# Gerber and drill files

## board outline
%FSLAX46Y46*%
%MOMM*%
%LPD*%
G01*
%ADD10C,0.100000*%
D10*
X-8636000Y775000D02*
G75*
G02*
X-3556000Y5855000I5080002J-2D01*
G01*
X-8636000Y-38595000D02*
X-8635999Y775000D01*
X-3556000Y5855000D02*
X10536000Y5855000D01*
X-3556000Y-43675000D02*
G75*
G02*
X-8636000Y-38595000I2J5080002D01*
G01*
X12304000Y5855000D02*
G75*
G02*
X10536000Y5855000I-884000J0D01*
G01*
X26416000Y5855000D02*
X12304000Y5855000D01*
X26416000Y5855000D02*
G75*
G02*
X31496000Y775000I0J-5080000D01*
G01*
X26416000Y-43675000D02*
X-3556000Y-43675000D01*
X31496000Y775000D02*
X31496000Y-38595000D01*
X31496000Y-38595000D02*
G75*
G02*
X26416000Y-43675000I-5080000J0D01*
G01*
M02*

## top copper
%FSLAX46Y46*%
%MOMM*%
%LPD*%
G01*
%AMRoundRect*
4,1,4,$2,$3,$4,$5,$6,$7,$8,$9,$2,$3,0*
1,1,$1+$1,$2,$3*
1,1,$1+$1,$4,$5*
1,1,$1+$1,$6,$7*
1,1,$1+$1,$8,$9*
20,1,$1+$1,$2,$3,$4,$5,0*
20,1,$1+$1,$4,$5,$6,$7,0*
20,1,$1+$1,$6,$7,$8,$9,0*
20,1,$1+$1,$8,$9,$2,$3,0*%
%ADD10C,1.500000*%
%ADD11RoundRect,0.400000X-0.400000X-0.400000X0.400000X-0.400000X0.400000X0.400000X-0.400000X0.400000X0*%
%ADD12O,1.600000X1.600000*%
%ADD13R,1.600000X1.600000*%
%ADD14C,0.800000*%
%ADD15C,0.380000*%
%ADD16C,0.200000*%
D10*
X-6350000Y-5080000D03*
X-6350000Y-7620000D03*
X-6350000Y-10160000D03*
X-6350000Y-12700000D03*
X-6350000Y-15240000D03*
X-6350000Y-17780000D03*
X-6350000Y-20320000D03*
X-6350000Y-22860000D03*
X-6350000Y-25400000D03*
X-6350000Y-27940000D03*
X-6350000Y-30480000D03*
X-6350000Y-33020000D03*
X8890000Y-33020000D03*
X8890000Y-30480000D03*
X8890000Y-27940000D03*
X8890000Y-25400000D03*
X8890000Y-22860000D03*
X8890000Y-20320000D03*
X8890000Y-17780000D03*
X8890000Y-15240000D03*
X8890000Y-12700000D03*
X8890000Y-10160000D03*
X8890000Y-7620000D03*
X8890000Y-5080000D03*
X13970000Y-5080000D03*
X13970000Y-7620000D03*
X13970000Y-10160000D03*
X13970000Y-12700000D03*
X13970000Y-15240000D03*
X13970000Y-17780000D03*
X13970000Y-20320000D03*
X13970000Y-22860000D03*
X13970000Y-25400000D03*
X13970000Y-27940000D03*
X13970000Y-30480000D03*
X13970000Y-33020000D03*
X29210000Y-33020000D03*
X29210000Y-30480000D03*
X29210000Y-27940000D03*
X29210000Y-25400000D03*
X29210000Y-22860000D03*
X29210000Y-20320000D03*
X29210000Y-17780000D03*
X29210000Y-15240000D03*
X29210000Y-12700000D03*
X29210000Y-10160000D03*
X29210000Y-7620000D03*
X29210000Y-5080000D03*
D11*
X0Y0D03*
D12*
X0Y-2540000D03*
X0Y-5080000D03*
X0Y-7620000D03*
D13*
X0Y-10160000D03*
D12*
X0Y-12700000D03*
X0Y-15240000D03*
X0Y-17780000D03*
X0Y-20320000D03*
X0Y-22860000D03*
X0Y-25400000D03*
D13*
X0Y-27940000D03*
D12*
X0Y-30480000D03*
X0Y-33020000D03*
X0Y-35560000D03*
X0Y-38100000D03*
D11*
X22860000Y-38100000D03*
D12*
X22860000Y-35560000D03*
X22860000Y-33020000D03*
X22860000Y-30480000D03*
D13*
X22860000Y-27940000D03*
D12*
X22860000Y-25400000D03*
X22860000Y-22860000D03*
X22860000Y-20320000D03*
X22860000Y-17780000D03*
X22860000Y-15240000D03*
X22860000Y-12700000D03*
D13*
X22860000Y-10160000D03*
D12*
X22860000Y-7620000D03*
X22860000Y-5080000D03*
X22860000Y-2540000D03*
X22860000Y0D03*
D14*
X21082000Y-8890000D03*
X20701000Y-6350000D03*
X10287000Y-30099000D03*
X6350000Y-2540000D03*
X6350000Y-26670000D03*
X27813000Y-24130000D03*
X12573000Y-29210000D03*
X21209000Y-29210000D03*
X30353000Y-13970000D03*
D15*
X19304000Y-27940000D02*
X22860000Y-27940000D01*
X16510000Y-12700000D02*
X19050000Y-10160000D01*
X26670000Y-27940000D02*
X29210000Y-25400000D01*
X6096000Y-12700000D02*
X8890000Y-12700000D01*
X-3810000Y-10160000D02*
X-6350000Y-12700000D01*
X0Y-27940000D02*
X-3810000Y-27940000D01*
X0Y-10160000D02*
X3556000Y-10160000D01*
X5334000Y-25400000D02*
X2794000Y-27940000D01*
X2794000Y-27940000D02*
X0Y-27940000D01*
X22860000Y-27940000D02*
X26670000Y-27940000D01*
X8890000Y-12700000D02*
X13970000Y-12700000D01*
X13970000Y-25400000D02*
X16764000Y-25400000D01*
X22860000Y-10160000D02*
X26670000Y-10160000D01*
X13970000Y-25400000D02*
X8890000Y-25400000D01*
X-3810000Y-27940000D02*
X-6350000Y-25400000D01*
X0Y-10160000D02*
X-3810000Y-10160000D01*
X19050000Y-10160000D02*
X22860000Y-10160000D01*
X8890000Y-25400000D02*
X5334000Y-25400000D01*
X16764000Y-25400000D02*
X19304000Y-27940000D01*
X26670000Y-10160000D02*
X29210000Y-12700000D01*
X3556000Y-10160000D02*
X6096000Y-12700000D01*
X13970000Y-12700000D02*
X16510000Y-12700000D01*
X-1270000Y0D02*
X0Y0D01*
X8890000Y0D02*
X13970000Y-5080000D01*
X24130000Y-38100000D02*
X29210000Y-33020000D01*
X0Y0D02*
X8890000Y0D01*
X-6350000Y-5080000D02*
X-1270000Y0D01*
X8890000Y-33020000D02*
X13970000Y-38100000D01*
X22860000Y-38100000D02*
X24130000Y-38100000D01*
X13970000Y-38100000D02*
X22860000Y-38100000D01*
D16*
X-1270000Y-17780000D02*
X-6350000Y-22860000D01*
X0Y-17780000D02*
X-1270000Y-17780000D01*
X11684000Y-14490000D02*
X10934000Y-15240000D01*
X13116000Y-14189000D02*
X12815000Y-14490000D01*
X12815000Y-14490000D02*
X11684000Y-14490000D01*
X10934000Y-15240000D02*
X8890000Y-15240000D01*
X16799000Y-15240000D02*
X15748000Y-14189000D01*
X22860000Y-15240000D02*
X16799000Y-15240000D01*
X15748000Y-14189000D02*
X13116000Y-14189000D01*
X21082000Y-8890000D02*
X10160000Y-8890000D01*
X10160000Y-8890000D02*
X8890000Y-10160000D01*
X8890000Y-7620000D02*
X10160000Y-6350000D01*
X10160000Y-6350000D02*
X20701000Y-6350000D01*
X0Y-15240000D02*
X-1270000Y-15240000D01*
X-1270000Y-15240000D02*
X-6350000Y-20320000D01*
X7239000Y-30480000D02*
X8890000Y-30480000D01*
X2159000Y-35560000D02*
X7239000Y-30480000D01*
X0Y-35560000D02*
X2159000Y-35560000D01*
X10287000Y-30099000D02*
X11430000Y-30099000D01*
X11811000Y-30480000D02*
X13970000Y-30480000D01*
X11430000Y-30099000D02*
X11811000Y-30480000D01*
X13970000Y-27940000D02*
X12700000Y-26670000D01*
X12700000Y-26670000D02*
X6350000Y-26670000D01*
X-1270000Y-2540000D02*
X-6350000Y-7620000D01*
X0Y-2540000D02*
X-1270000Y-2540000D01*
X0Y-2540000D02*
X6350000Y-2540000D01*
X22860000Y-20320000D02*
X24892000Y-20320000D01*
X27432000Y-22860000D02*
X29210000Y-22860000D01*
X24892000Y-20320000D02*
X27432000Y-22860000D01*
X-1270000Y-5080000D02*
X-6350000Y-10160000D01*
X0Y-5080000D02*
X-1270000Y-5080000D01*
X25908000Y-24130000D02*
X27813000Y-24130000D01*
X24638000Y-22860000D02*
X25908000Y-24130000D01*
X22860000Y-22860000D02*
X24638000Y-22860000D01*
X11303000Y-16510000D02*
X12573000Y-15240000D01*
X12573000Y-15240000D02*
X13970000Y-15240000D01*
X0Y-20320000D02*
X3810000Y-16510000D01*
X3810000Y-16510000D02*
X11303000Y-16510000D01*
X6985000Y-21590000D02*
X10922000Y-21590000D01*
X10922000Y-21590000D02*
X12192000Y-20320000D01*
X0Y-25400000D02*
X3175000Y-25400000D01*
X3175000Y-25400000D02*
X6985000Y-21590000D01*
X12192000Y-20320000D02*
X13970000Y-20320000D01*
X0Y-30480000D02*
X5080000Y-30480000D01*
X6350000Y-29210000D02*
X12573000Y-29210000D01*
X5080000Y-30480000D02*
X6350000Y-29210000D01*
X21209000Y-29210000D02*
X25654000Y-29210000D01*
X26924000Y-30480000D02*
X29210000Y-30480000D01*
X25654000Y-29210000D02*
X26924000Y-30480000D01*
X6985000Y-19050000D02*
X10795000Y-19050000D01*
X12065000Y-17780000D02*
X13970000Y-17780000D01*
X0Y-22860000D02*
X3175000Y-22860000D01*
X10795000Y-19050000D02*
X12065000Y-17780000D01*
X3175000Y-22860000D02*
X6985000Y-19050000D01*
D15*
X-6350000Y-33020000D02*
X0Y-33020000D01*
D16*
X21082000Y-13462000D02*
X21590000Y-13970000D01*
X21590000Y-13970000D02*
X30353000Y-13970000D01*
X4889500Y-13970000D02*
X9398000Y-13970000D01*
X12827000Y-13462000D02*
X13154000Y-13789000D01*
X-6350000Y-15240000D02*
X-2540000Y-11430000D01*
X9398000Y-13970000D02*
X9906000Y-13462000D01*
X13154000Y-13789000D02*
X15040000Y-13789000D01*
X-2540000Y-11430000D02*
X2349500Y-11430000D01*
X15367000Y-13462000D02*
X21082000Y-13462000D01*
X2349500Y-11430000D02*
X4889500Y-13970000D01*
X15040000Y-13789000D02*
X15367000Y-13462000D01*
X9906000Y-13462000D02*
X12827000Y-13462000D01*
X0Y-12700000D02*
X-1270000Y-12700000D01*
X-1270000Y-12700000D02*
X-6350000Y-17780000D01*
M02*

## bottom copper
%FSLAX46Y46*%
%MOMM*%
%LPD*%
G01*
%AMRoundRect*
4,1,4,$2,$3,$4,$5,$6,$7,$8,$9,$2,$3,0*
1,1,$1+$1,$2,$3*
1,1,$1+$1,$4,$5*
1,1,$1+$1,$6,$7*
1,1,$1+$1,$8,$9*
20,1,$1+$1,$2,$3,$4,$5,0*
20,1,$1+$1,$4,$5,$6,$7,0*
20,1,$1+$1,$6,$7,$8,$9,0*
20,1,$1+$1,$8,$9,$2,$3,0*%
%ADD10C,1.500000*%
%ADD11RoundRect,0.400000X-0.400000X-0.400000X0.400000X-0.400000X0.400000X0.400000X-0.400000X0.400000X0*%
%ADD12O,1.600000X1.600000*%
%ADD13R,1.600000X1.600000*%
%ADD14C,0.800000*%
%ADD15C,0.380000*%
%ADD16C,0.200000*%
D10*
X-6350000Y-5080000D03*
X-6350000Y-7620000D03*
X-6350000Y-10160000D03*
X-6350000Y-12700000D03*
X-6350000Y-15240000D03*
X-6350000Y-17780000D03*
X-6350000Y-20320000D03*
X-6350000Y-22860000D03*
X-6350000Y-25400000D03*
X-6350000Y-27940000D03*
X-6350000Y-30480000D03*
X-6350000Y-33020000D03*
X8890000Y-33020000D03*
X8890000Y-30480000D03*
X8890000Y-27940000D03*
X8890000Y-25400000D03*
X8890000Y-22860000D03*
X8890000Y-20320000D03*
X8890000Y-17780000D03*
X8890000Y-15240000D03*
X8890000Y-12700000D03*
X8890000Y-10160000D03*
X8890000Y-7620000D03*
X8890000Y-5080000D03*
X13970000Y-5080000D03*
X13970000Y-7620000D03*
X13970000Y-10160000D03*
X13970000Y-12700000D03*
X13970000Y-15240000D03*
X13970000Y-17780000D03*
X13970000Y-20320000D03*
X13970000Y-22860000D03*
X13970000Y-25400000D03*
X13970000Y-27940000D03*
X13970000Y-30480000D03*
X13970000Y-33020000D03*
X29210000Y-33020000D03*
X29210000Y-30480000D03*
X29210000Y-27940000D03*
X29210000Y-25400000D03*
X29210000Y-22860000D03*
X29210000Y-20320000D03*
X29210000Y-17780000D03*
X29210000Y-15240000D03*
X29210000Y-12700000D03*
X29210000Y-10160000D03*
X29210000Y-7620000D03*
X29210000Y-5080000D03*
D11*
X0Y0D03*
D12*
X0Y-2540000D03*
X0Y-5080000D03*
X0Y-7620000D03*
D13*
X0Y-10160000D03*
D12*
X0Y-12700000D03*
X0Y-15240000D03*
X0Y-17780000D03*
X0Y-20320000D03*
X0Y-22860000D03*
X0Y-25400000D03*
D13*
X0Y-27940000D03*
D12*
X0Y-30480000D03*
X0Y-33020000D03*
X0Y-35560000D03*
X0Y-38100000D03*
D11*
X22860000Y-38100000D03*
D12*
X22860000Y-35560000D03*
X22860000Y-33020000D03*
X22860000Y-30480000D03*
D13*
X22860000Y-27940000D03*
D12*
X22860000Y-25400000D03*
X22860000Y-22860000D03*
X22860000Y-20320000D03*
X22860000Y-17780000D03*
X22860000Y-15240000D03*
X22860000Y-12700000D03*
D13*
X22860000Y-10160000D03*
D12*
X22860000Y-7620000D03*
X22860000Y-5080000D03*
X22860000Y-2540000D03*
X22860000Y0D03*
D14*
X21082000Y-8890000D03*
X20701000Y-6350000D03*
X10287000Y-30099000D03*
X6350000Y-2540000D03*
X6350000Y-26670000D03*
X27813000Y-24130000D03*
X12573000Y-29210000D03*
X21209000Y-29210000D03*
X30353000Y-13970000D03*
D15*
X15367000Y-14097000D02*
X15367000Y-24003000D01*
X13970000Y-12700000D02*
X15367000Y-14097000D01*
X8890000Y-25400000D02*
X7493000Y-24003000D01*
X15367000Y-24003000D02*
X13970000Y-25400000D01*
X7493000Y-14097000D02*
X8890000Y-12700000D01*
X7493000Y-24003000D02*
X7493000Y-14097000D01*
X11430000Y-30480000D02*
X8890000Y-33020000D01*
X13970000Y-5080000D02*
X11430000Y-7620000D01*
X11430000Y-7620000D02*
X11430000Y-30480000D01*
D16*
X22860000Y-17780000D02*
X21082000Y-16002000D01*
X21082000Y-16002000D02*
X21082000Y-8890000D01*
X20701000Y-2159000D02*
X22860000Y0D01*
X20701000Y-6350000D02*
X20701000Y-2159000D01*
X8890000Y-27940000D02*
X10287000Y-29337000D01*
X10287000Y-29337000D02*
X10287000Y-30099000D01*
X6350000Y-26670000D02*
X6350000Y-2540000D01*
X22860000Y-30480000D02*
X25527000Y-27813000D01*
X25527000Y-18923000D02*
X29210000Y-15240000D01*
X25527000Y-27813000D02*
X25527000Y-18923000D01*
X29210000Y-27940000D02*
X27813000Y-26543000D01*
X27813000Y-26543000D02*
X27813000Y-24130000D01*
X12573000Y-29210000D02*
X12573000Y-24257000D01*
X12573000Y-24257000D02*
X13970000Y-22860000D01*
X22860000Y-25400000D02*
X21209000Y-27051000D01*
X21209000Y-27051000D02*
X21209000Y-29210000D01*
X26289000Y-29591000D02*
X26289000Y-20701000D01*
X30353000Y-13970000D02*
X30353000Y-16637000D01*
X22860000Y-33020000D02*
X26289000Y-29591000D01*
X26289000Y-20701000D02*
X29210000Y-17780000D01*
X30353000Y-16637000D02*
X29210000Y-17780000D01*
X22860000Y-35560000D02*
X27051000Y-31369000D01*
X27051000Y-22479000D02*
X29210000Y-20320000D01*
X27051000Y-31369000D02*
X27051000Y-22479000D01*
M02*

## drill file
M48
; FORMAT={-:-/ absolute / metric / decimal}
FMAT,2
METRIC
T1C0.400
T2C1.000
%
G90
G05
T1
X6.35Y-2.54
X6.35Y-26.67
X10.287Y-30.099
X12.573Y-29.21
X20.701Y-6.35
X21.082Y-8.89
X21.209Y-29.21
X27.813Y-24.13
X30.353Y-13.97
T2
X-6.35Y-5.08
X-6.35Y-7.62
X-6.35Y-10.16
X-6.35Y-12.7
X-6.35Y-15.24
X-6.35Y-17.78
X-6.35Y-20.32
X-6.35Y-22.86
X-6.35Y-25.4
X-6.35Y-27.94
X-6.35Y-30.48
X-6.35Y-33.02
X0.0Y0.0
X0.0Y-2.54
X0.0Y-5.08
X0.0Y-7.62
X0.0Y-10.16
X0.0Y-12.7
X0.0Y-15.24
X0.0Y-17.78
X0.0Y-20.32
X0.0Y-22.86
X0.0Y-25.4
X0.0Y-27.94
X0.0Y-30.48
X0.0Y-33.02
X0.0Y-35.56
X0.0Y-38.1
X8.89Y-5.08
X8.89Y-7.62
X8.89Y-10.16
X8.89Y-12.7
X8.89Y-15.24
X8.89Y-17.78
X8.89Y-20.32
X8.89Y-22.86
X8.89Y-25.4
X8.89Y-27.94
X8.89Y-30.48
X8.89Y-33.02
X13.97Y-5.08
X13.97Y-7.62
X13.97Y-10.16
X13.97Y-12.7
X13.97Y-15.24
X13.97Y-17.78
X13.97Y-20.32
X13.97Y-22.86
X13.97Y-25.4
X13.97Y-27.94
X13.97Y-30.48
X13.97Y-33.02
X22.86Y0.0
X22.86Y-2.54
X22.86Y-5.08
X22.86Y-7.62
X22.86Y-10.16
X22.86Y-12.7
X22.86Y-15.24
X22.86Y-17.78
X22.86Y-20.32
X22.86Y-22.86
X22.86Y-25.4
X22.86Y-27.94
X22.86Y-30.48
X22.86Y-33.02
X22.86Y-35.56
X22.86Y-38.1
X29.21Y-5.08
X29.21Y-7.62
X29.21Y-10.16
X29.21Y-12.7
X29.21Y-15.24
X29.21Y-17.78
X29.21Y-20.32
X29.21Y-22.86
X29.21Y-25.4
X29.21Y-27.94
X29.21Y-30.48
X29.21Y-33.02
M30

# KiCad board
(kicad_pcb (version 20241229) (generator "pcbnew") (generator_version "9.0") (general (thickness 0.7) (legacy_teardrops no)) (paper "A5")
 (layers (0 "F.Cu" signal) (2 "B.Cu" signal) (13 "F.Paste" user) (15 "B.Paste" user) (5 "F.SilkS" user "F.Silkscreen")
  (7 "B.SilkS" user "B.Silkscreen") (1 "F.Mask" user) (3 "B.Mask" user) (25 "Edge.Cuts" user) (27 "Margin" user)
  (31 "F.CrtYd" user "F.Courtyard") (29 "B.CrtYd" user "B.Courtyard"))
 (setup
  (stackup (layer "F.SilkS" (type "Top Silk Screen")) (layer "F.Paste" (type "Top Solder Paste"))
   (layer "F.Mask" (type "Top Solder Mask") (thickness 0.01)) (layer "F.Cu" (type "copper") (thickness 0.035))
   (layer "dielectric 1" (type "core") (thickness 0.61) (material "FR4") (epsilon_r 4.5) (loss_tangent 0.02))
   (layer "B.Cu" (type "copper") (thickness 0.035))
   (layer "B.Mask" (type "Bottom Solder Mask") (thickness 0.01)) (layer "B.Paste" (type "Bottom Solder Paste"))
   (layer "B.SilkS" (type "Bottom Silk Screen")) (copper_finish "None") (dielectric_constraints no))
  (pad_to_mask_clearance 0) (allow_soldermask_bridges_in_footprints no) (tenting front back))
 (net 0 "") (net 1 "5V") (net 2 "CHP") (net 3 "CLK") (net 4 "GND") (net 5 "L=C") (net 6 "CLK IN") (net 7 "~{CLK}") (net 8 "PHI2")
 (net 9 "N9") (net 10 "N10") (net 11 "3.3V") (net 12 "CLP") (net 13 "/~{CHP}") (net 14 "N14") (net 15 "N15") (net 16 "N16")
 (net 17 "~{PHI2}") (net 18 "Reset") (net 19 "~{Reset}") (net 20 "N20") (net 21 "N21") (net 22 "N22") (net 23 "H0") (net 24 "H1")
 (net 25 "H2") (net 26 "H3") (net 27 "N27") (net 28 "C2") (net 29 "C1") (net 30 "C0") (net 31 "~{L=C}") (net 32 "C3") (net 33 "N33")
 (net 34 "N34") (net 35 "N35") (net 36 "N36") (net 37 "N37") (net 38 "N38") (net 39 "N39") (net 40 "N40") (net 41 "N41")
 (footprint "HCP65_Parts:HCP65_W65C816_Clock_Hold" (layer "F.Cu") (at -6.35 5.08)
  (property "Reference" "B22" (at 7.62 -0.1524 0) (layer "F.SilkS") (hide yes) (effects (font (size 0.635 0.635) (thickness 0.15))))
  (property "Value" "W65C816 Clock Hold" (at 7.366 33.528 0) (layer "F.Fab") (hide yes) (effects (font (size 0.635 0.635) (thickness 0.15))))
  (pad "1" thru_hole circle (at 0 0) (size 1.5 1.5) (drill 1) (layers "*.Cu" "*.Mask") (remove_unused_layers no) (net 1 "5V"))
  (pad "2" thru_hole circle (at 0 2.54) (size 1.5 1.5) (drill 1) (layers "*.Cu" "*.Mask") (remove_unused_layers no) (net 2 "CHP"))
  (pad "3" thru_hole circle (at 0 5.08) (size 1.5 1.5) (drill 1) (layers "*.Cu" "*.Mask") (remove_unused_layers no) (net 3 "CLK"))
  (pad "4" thru_hole circle (at 0 7.62) (size 1.5 1.5) (drill 1) (layers "*.Cu" "*.Mask") (remove_unused_layers no) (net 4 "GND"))
  (pad "5" thru_hole circle (at 0 10.16) (size 1.5 1.5) (drill 1) (layers "*.Cu" "*.Mask") (remove_unused_layers no) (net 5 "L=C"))
  (pad "6" thru_hole circle (at 0 12.7) (size 1.5 1.5) (drill 1) (layers "*.Cu" "*.Mask") (remove_unused_layers no) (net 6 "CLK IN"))
  (pad "7" thru_hole circle (at 0 15.24) (size 1.5 1.5) (drill 1) (layers "*.Cu" "*.Mask") (remove_unused_layers no) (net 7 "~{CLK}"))
  (pad "8" thru_hole circle (at 0 17.78) (size 1.5 1.5) (drill 1) (layers "*.Cu" "*.Mask") (remove_unused_layers no) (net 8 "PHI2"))
  (pad "9" thru_hole circle (at 0 20.32) (size 1.5 1.5) (drill 1) (layers "*.Cu" "*.Mask") (remove_unused_layers no) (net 4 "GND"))
  (pad "10" thru_hole circle (at 0 22.86) (size 1.5 1.5) (drill 1) (layers "*.Cu" "*.Mask") (remove_unused_layers no) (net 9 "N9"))
  (pad "11" thru_hole circle (at 0 25.4) (size 1.5 1.5) (drill 1) (layers "*.Cu" "*.Mask") (remove_unused_layers no) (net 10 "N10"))
  (pad "12" thru_hole circle (at 0 27.94) (size 1.5 1.5) (drill 1) (layers "*.Cu" "*.Mask") (remove_unused_layers no) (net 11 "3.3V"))
  (pad "13" thru_hole circle (at 15.24 27.94) (size 1.5 1.5) (drill 1) (layers "*.Cu" "*.Mask") (remove_unused_layers no) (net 1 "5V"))
  (pad "14" thru_hole circle (at 15.24 25.4) (size 1.5 1.5) (drill 1) (layers "*.Cu" "*.Mask") (remove_unused_layers no) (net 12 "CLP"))
  (pad "15" thru_hole circle (at 15.24 22.86) (size 1.5 1.5) (drill 1) (layers "*.Cu" "*.Mask") (remove_unused_layers no) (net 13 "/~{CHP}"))
  (pad "16" thru_hole circle (at 15.24 20.32) (size 1.5 1.5) (drill 1) (layers "*.Cu" "*.Mask") (remove_unused_layers no) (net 4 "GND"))
  (pad "17" thru_hole circle (at 15.24 17.78) (size 1.5 1.5) (drill 1) (layers "*.Cu" "*.Mask") (remove_unused_layers no) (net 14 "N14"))
  (pad "18" thru_hole circle (at 15.24 15.24) (size 1.5 1.5) (drill 1) (layers "*.Cu" "*.Mask") (remove_unused_layers no) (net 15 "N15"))
  (pad "19" thru_hole circle (at 15.24 12.7) (size 1.5 1.5) (drill 1) (layers "*.Cu" "*.Mask") (remove_unused_layers no) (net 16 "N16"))
  (pad "20" thru_hole circle (at 15.24 10.16) (size 1.5 1.5) (drill 1) (layers "*.Cu" "*.Mask") (remove_unused_layers no) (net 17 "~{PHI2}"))
  (pad "21" thru_hole circle (at 15.24 7.62) (size 1.5 1.5) (drill 1) (layers "*.Cu" "*.Mask") (remove_unused_layers no) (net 4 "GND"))
  (pad "22" thru_hole circle (at 15.24 5.08) (size 1.5 1.5) (drill 1) (layers "*.Cu" "*.Mask") (remove_unused_layers no) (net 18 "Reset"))
  (pad "23" thru_hole circle (at 15.24 2.54) (size 1.5 1.5) (drill 1) (layers "*.Cu" "*.Mask") (remove_unused_layers no) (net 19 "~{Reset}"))
  (pad "24" thru_hole circle (at 15.24 0) (size 1.5 1.5) (drill 1) (layers "*.Cu" "*.Mask") (remove_unused_layers no) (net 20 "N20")))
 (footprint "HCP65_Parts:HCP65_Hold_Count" (layer "F.Cu") (at 13.97 5.08)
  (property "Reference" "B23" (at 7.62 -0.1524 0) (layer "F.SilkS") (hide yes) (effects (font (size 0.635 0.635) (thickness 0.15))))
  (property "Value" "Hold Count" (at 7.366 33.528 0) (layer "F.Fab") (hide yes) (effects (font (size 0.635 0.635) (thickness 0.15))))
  (pad "1" thru_hole circle (at 0 0) (size 1.5 1.5) (drill 1) (layers "*.Cu" "*.Mask") (remove_unused_layers no) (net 1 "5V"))
  (pad "2" thru_hole circle (at 0 2.54) (size 1.5 1.5) (drill 1) (layers "*.Cu" "*.Mask") (remove_unused_layers no) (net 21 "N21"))
  (pad "3" thru_hole circle (at 0 5.08) (size 1.5 1.5) (drill 1) (layers "*.Cu" "*.Mask") (remove_unused_layers no) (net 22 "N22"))
  (pad "4" thru_hole circle (at 0 7.62) (size 1.5 1.5) (drill 1) (layers "*.Cu" "*.Mask") (remove_unused_layers no) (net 4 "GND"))
  (pad "5" thru_hole circle (at 0 10.16) (size 1.5 1.5) (drill 1) (layers "*.Cu" "*.Mask") (remove_unused_layers no) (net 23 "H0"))
  (pad "6" thru_hole circle (at 0 12.7) (size 1.5 1.5) (drill 1) (layers "*.Cu" "*.Mask") (remove_unused_layers no) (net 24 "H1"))
  (pad "7" thru_hole circle (at 0 15.24) (size 1.5 1.5) (drill 1) (layers "*.Cu" "*.Mask") (remove_unused_layers no) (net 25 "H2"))
  (pad "8" thru_hole circle (at 0 17.78) (size 1.5 1.5) (drill 1) (layers "*.Cu" "*.Mask") (remove_unused_layers no) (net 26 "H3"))
  (pad "9" thru_hole circle (at 0 20.32) (size 1.5 1.5) (drill 1) (layers "*.Cu" "*.Mask") (remove_unused_layers no) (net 4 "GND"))
  (pad "10" thru_hole circle (at 0 22.86) (size 1.5 1.5) (drill 1) (layers "*.Cu" "*.Mask") (remove_unused_layers no) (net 2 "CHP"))
  (pad "11" thru_hole circle (at 0 25.4) (size 1.5 1.5) (drill 1) (layers "*.Cu" "*.Mask") (remove_unused_layers no) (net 13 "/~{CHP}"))
  (pad "12" thru_hole circle (at 0 27.94) (size 1.5 1.5) (drill 1) (layers "*.Cu" "*.Mask") (remove_unused_layers no) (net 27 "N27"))
  (pad "13" thru_hole circle (at 15.24 27.94) (size 1.5 1.5) (drill 1) (layers "*.Cu" "*.Mask") (remove_unused_layers no) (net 1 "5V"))
  (pad "14" thru_hole circle (at 15.24 25.4) (size 1.5 1.5) (drill 1) (layers "*.Cu" "*.Mask") (remove_unused_layers no) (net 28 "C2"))
  (pad "15" thru_hole circle (at 15.24 22.86) (size 1.5 1.5) (drill 1) (layers "*.Cu" "*.Mask") (remove_unused_layers no) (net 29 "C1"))
  (pad "16" thru_hole circle (at 15.24 20.32) (size 1.5 1.5) (drill 1) (layers "*.Cu" "*.Mask") (remove_unused_layers no) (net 4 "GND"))
  (pad "17" thru_hole circle (at 15.24 17.78) (size 1.5 1.5) (drill 1) (layers "*.Cu" "*.Mask") (remove_unused_layers no) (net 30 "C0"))
  (pad "18" thru_hole circle (at 15.24 15.24) (size 1.5 1.5) (drill 1) (layers "*.Cu" "*.Mask") (remove_unused_layers no) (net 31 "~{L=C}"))
  (pad "19" thru_hole circle (at 15.24 12.7) (size 1.5 1.5) (drill 1) (layers "*.Cu" "*.Mask") (remove_unused_layers no) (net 5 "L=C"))
  (pad "20" thru_hole circle (at 15.24 10.16) (size 1.5 1.5) (drill 1) (layers "*.Cu" "*.Mask") (remove_unused_layers no) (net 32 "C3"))
  (pad "21" thru_hole circle (at 15.24 7.62) (size 1.5 1.5) (drill 1) (layers "*.Cu" "*.Mask") (remove_unused_layers no) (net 4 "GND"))
  (pad "22" thru_hole circle (at 15.24 5.08) (size 1.5 1.5) (drill 1) (layers "*.Cu" "*.Mask") (remove_unused_layers no) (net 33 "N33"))
  (pad "23" thru_hole circle (at 15.24 2.54) (size 1.5 1.5) (drill 1) (layers "*.Cu" "*.Mask") (remove_unused_layers no) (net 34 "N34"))
  (pad "24" thru_hole circle (at 15.24 0) (size 1.5 1.5) (drill 1) (layers "*.Cu" "*.Mask") (remove_unused_layers no) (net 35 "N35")))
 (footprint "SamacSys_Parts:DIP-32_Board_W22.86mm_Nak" (layer "F.Cu") (at 0 0)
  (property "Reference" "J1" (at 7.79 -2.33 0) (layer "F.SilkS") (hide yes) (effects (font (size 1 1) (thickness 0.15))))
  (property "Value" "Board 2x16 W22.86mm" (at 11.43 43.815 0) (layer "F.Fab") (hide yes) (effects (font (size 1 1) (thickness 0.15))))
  (pad "1" thru_hole roundrect (at 0 0) (size 1.6 1.6) (drill 1) (layers "*.Cu" "*.Mask") (remove_unused_layers no) (roundrect_rratio 0.25)
   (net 1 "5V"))
  (pad "2" thru_hole oval (at 0 2.54) (size 1.6 1.6) (drill 1) (layers "*.Cu" "*.Mask") (remove_unused_layers no) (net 2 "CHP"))
  (pad "3" thru_hole oval (at 0 5.08) (size 1.6 1.6) (drill 1) (layers "*.Cu" "*.Mask") (remove_unused_layers no) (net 3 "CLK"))
  (pad "4" thru_hole oval (at 0 7.62) (size 1.6 1.6) (drill 1) (layers "*.Cu" "*.Mask") (remove_unused_layers no) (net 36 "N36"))
  (pad "5" thru_hole rect (at 0 10.16) (size 1.6 1.6) (drill 1) (layers "*.Cu" "*.Mask") (remove_unused_layers no) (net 4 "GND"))
  (pad "6" thru_hole oval (at 0 12.7) (size 1.6 1.6) (drill 1) (layers "*.Cu" "*.Mask") (remove_unused_layers no) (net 6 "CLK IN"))
  (pad "7" thru_hole oval (at 0 15.24) (size 1.6 1.6) (drill 1) (layers "*.Cu" "*.Mask") (remove_unused_layers no) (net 7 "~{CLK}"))
  (pad "8" thru_hole oval (at 0 17.78) (size 1.6 1.6) (drill 1) (layers "*.Cu" "*.Mask") (remove_unused_layers no) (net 8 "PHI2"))
  (pad "9" thru_hole oval (at 0 20.32) (size 1.6 1.6) (drill 1) (layers "*.Cu" "*.Mask") (remove_unused_layers no) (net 23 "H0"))
  (pad "10" thru_hole oval (at 0 22.86) (size 1.6 1.6) (drill 1) (layers "*.Cu" "*.Mask") (remove_unused_layers no) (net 24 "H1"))
  (pad "11" thru_hole oval (at 0 25.4) (size 1.6 1.6) (drill 1) (layers "*.Cu" "*.Mask") (remove_unused_layers no) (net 25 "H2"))
  (pad "12" thru_hole rect (at 0 27.94) (size 1.6 1.6) (drill 1) (layers "*.Cu" "*.Mask") (remove_unused_layers no) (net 4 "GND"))
  (pad "13" thru_hole oval (at 0 30.48) (size 1.6 1.6) (drill 1) (layers "*.Cu" "*.Mask") (remove_unused_layers no) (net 26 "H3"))
  (pad "14" thru_hole oval (at 0 33.02) (size 1.6 1.6) (drill 1) (layers "*.Cu" "*.Mask") (remove_unused_layers no) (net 11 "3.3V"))
  (pad "15" thru_hole oval (at 0 35.56) (size 1.6 1.6) (drill 1) (layers "*.Cu" "*.Mask") (remove_unused_layers no) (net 12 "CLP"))
  (pad "16" thru_hole oval (at 0 38.1) (size 1.6 1.6) (drill 1) (layers "*.Cu" "*.Mask") (remove_unused_layers no) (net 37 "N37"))
  (pad "17" thru_hole roundrect (at 22.86 38.1) (size 1.6 1.6) (drill 1) (layers "*.Cu" "*.Mask") (remove_unused_layers no)
   (roundrect_rratio 0.25) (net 1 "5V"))
  (pad "18" thru_hole oval (at 22.86 35.56) (size 1.6 1.6) (drill 1) (layers "*.Cu" "*.Mask") (remove_unused_layers no) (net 31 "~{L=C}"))
  (pad "19" thru_hole oval (at 22.86 33.02) (size 1.6 1.6) (drill 1) (layers "*.Cu" "*.Mask") (remove_unused_layers no) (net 5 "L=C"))
  (pad "20" thru_hole oval (at 22.86 30.48) (size 1.6 1.6) (drill 1) (layers "*.Cu" "*.Mask") (remove_unused_layers no) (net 32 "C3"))
  (pad "21" thru_hole rect (at 22.86 27.94) (size 1.6 1.6) (drill 1) (layers "*.Cu" "*.Mask") (remove_unused_layers no) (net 4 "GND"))
  (pad "22" thru_hole oval (at 22.86 25.4) (size 1.6 1.6) (drill 1) (layers "*.Cu" "*.Mask") (remove_unused_layers no) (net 28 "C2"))
  (pad "23" thru_hole oval (at 22.86 22.86) (size 1.6 1.6) (drill 1) (layers "*.Cu" "*.Mask") (remove_unused_layers no) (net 29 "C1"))
  (pad "24" thru_hole oval (at 22.86 20.32) (size 1.6 1.6) (drill 1) (layers "*.Cu" "*.Mask") (remove_unused_layers no) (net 30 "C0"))
  (pad "25" thru_hole oval (at 22.86 17.78) (size 1.6 1.6) (drill 1) (layers "*.Cu" "*.Mask") (remove_unused_layers no) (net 18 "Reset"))
  (pad "26" thru_hole oval (at 22.86 15.24) (size 1.6 1.6) (drill 1) (layers "*.Cu" "*.Mask") (remove_unused_layers no) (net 17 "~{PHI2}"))
  (pad "27" thru_hole oval (at 22.86 12.7) (size 1.6 1.6) (drill 1) (layers "*.Cu" "*.Mask") (remove_unused_layers no) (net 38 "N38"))
  (pad "28" thru_hole rect (at 22.86 10.16) (size 1.6 1.6) (drill 1) (layers "*.Cu" "*.Mask") (remove_unused_layers no) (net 4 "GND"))
  (pad "29" thru_hole oval (at 22.86 7.62) (size 1.6 1.6) (drill 1) (layers "*.Cu" "*.Mask") (remove_unused_layers no) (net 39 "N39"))
  (pad "30" thru_hole oval (at 22.86 5.08) (size 1.6 1.6) (drill 1) (layers "*.Cu" "*.Mask") (remove_unused_layers no) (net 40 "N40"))
  (pad "31" thru_hole oval (at 22.86 2.54) (size 1.6 1.6) (drill 1) (layers "*.Cu" "*.Mask") (remove_unused_layers no) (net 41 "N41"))
  (pad "32" thru_hole oval (at 22.86 0) (size 1.6 1.6) (drill 1) (layers "*.Cu" "*.Mask") (remove_unused_layers no) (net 19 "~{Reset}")))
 (gr_arc (start -8.636 -0.775) (mid -7.148102 -4.367102) (end -3.556 -5.855) (stroke (width 0.1) (type default)) (layer "Edge.Cuts"))
 (gr_line (start -8.636 38.595) (end -8.635999 -0.775) (stroke (width 0.1) (type default)) (layer "Edge.Cuts"))
 (gr_line (start -3.556 -5.855) (end 10.536 -5.855) (stroke (width 0.1) (type default)) (layer "Edge.Cuts"))
 (gr_arc (start -3.556 43.675) (mid -7.148102 42.187102) (end -8.636 38.595) (stroke (width 0.1) (type default)) (layer "Edge.Cuts"))
 (gr_arc (start 12.304 -5.855) (mid 11.42 -4.971) (end 10.536 -5.855) (stroke (width 0.1) (type solid)) (layer "Edge.Cuts"))
 (gr_line (start 26.416 -5.855) (end 12.304 -5.855) (stroke (width 0.1) (type solid)) (layer "Edge.Cuts"))
 (gr_arc (start 26.416 -5.855) (mid 30.008102 -4.367102) (end 31.496 -0.775) (stroke (width 0.1) (type default)) (layer "Edge.Cuts"))
 (gr_line (start 26.416 43.675) (end -3.556 43.675) (stroke (width 0.1) (type default)) (layer "Edge.Cuts"))
 (gr_line (start 31.496 -0.775) (end 31.496 38.595) (stroke (width 0.1) (type default)) (layer "Edge.Cuts"))
 (gr_arc (start 31.496 38.595) (mid 30.008102 42.187102) (end 26.416 43.675) (stroke (width 0.1) (type default)) (layer "Edge.Cuts"))
 (segment (start 19.304 27.94) (end 22.86 27.94) (width 0.38) (layer "F.Cu") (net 4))
 (segment (start 16.51 12.7) (end 19.05 10.16) (width 0.38) (layer "F.Cu") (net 4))
 (segment (start 26.67 27.94) (end 29.21 25.4) (width 0.38) (layer "F.Cu") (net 4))
 (segment (start 6.096 12.7) (end 8.89 12.7) (width 0.38) (layer "F.Cu") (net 4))
 (segment (start -3.81 10.16) (end -6.35 12.7) (width 0.38) (layer "F.Cu") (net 4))
 (segment (start 0 27.94) (end -3.81 27.94) (width 0.38) (layer "F.Cu") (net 4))
 (segment (start 0 10.16) (end 3.556 10.16) (width 0.38) (layer "F.Cu") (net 4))
 (segment (start 5.334 25.4) (end 2.794 27.94) (width 0.38) (layer "F.Cu") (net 4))
 (segment (start 2.794 27.94) (end 0 27.94) (width 0.38) (layer "F.Cu") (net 4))
 (segment (start 22.86 27.94) (end 26.67 27.94) (width 0.38) (layer "F.Cu") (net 4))
 (segment (start 8.89 12.7) (end 13.97 12.7) (width 0.38) (layer "F.Cu") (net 4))
 (segment (start 13.97 25.4) (end 16.764 25.4) (width 0.38) (layer "F.Cu") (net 4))
 (segment (start 22.86 10.16) (end 26.67 10.16) (width 0.38) (layer "F.Cu") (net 4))
 (segment (start 13.97 25.4) (end 8.89 25.4) (width 0.38) (layer "F.Cu") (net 4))
 (segment (start -3.81 27.94) (end -6.35 25.4) (width 0.38) (layer "F.Cu") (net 4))
 (segment (start 0 10.16) (end -3.81 10.16) (width 0.38) (layer "F.Cu") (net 4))
 (segment (start 19.05 10.16) (end 22.86 10.16) (width 0.38) (layer "F.Cu") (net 4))
 (segment (start 8.89 25.4) (end 5.334 25.4) (width 0.38) (layer "F.Cu") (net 4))
 (segment (start 16.764 25.4) (end 19.304 27.94) (width 0.38) (layer "F.Cu") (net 4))
 (segment (start 26.67 10.16) (end 29.21 12.7) (width 0.38) (layer "F.Cu") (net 4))
 (segment (start 3.556 10.16) (end 6.096 12.7) (width 0.38) (layer "F.Cu") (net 4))
 (segment (start 13.97 12.7) (end 16.51 12.7) (width 0.38) (layer "F.Cu") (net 4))
 (segment (start 15.367 14.097) (end 15.367 24.003) (width 0.38) (layer "B.Cu") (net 4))
 (segment (start 13.97 12.7) (end 15.367 14.097) (width 0.38) (layer "B.Cu") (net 4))
 (segment (start 8.89 25.4) (end 7.493 24.003) (width 0.38) (layer "B.Cu") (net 4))
 (segment (start 15.367 24.003) (end 13.97 25.4) (width 0.38) (layer "B.Cu") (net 4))
 (segment (start 7.493 14.097) (end 8.89 12.7) (width 0.38) (layer "B.Cu") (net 4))
 (segment (start 7.493 24.003) (end 7.493 14.097) (width 0.38) (layer "B.Cu") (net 4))
 (segment (start -1.27 0) (end 0 0) (width 0.38) (layer "F.Cu") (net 1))
 (segment (start 8.89 0) (end 13.97 5.08) (width 0.38) (layer "F.Cu") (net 1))
 (segment (start 24.13 38.1) (end 29.21 33.02) (width 0.38) (layer "F.Cu") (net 1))
 (segment (start 0 0) (end 8.89 0) (width 0.38) (layer "F.Cu") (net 1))
 (segment (start -6.35 5.08) (end -1.27 0) (width 0.38) (layer "F.Cu") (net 1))
 (segment (start 8.89 33.02) (end 13.97 38.1) (width 0.38) (layer "F.Cu") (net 1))
 (segment (start 22.86 38.1) (end 24.13 38.1) (width 0.38) (layer "F.Cu") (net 1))
 (segment (start 13.97 38.1) (end 22.86 38.1) (width 0.38) (layer "F.Cu") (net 1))
 (segment (start 11.43 30.48) (end 8.89 33.02) (width 0.38) (layer "B.Cu") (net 1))
 (segment (start 13.97 5.08) (end 11.43 7.62) (width 0.38) (layer "B.Cu") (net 1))
 (segment (start 11.43 7.62) (end 11.43 30.48) (width 0.38) (layer "B.Cu") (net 1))
 (segment (start -1.27 17.78) (end -6.35 22.86) (width 0.2) (layer "F.Cu") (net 8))
 (segment (start 0 17.78) (end -1.27 17.78) (width 0.2) (layer "F.Cu") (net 8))
 (segment (start 11.684 14.49) (end 10.934 15.24) (width 0.2) (layer "F.Cu") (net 17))
 (segment (start 13.116 14.189) (end 12.815 14.49) (width 0.2) (layer "F.Cu") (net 17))
 (segment (start 12.815 14.49) (end 11.684 14.49) (width 0.2) (layer "F.Cu") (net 17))
 (segment (start 10.934 15.24) (end 8.89 15.24) (width 0.2) (layer "F.Cu") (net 17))
 (segment (start 16.799 15.24) (end 15.748 14.189) (width 0.2) (layer "F.Cu") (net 17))
 (segment (start 22.86 15.24) (end 16.799 15.24) (width 0.2) (layer "F.Cu") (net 17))
 (segment (start 15.748 14.189) (end 13.116 14.189) (width 0.2) (layer "F.Cu") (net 17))
 (segment (start 21.082 8.89) (end 10.16 8.89) (width 0.2) (layer "F.Cu") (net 18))
 (segment (start 10.16 8.89) (end 8.89 10.16) (width 0.2) (layer "F.Cu") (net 18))
 (via (at 21.082 8.89) (size 0.8) (drill 0.4) (layers "F.Cu" "B.Cu") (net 18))
 (segment (start 22.86 17.78) (end 21.082 16.002) (width 0.2) (layer "B.Cu") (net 18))
 (segment (start 21.082 16.002) (end 21.082 8.89) (width 0.2) (layer "B.Cu") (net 18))
 (segment (start 8.89 7.62) (end 10.16 6.35) (width 0.2) (layer "F.Cu") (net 19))
 (segment (start 10.16 6.35) (end 20.701 6.35) (width 0.2) (layer "F.Cu") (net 19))
 (via (at 20.701 6.35) (size 0.8) (drill 0.4) (layers "F.Cu" "B.Cu") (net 19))
 (segment (start 20.701 2.159) (end 22.86 0) (width 0.2) (layer "B.Cu") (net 19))
 (segment (start 20.701 6.35) (end 20.701 2.159) (width 0.2) (layer "B.Cu") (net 19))
 (segment (start 0 15.24) (end -1.27 15.24) (width 0.2) (layer "F.Cu") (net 7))
 (segment (start -1.27 15.24) (end -6.35 20.32) (width 0.2) (layer "F.Cu") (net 7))
 (segment (start 7.239 30.48) (end 8.89 30.48) (width 0.2) (layer "F.Cu") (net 12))
 (segment (start 2.159 35.56) (end 7.239 30.48) (width 0.2) (layer "F.Cu") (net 12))
 (segment (start 0 35.56) (end 2.159 35.56) (width 0.2) (layer "F.Cu") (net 12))
 (segment (start 10.287 30.099) (end 11.43 30.099) (width 0.2) (layer "F.Cu") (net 13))
 (segment (start 11.811 30.48) (end 13.97 30.48) (width 0.2) (layer "F.Cu") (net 13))
 (segment (start 11.43 30.099) (end 11.811 30.48) (width 0.2) (layer "F.Cu") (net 13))
 (via (at 10.287 30.099) (size 0.8) (drill 0.4) (layers "F.Cu" "B.Cu") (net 13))
 (segment (start 8.89 27.94) (end 10.287 29.337) (width 0.2) (layer "B.Cu") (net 13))
 (segment (start 10.287 29.337) (end 10.287 30.099) (width 0.2) (layer "B.Cu") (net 13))
 (segment (start 13.97 27.94) (end 12.7 26.67) (width 0.2) (layer "F.Cu") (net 2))
 (segment (start 12.7 26.67) (end 6.35 26.67) (width 0.2) (layer "F.Cu") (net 2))
 (segment (start -1.27 2.54) (end -6.35 7.62) (width 0.2) (layer "F.Cu") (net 2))
 (segment (start 0 2.54) (end -1.27 2.54) (width 0.2) (layer "F.Cu") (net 2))
 (segment (start 0 2.54) (end 6.35 2.54) (width 0.2) (layer "F.Cu") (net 2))
 (via (at 6.35 2.54) (size 0.8) (drill 0.4) (layers "F.Cu" "B.Cu") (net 2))
 (via (at 6.35 26.67) (size 0.8) (drill 0.4) (layers "F.Cu" "B.Cu") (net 2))
 (segment (start 6.35 26.67) (end 6.35 2.54) (width 0.2) (layer "B.Cu") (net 2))
 (segment (start 22.86 20.32) (end 24.892 20.32) (width 0.2) (layer "F.Cu") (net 30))
 (segment (start 27.432 22.86) (end 29.21 22.86) (width 0.2) (layer "F.Cu") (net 30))
 (segment (start 24.892 20.32) (end 27.432 22.86) (width 0.2) (layer "F.Cu") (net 30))
 (segment (start -1.27 5.08) (end -6.35 10.16) (width 0.2) (layer "F.Cu") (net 3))
 (segment (start 0 5.08) (end -1.27 5.08) (width 0.2) (layer "F.Cu") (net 3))
 (segment (start 22.86 30.48) (end 25.527 27.813) (width 0.2) (layer "B.Cu") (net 32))
 (segment (start 25.527 18.923) (end 29.21 15.24) (width 0.2) (layer "B.Cu") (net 32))
 (segment (start 25.527 27.813) (end 25.527 18.923) (width 0.2) (layer "B.Cu") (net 32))
 (segment (start 25.908 24.13) (end 27.813 24.13) (width 0.2) (layer "F.Cu") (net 29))
 (segment (start 24.638 22.86) (end 25.908 24.13) (width 0.2) (layer "F.Cu") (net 29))
 (segment (start 22.86 22.86) (end 24.638 22.86) (width 0.2) (layer "F.Cu") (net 29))
 (via (at 27.813 24.13) (size 0.8) (drill 0.4) (layers "F.Cu" "B.Cu") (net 29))
 (segment (start 29.21 27.94) (end 27.813 26.543) (width 0.2) (layer "B.Cu") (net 29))
 (segment (start 27.813 26.543) (end 27.813 24.13) (width 0.2) (layer "B.Cu") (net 29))
 (segment (start 11.303 16.51) (end 12.573 15.24) (width 0.2) (layer "F.Cu") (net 23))
 (segment (start 12.573 15.24) (end 13.97 15.24) (width 0.2) (layer "F.Cu") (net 23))
 (segment (start 0 20.32) (end 3.81 16.51) (width 0.2) (layer "F.Cu") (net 23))
 (segment (start 3.81 16.51) (end 11.303 16.51) (width 0.2) (layer "F.Cu") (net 23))
 (segment (start 6.985 21.59) (end 10.922 21.59) (width 0.2) (layer "F.Cu") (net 25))
 (segment (start 10.922 21.59) (end 12.192 20.32) (width 0.2) (layer "F.Cu") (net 25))
 (segment (start 0 25.4) (end 3.175 25.4) (width 0.2) (layer "F.Cu") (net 25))
 (segment (start 3.175 25.4) (end 6.985 21.59) (width 0.2) (layer "F.Cu") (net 25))
 (segment (start 12.192 20.32) (end 13.97 20.32) (width 0.2) (layer "F.Cu") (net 25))
 (segment (start 0 30.48) (end 5.08 30.48) (width 0.2) (layer "F.Cu") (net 26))
 (segment (start 6.35 29.21) (end 12.573 29.21) (width 0.2) (layer "F.Cu") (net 26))
 (segment (start 5.08 30.48) (end 6.35 29.21) (width 0.2) (layer "F.Cu") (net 26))
 (via (at 12.573 29.21) (size 0.8) (drill 0.4) (layers "F.Cu" "B.Cu") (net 26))
 (segment (start 12.573 29.21) (end 12.573 24.257) (width 0.2) (layer "B.Cu") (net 26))
 (segment (start 12.573 24.257) (end 13.97 22.86) (width 0.2) (layer "B.Cu") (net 26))
 (segment (start 21.209 29.21) (end 25.654 29.21) (width 0.2) (layer "F.Cu") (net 28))
 (segment (start 26.924 30.48) (end 29.21 30.48) (width 0.2) (layer "F.Cu") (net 28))
 (segment (start 25.654 29.21) (end 26.924 30.48) (width 0.2) (layer "F.Cu") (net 28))
 (via (at 21.209 29.21) (size 0.8) (drill 0.4) (layers "F.Cu" "B.Cu") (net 28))
 (segment (start 22.86 25.4) (end 21.209 27.051) (width 0.2) (layer "B.Cu") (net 28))
 (segment (start 21.209 27.051) (end 21.209 29.21) (width 0.2) (layer "B.Cu") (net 28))
 (segment (start 6.985 19.05) (end 10.795 19.05) (width 0.2) (layer "F.Cu") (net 24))
 (segment (start 12.065 17.78) (end 13.97 17.78) (width 0.2) (layer "F.Cu") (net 24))
 (segment (start 0 22.86) (end 3.175 22.86) (width 0.2) (layer "F.Cu") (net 24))
 (segment (start 10.795 19.05) (end 12.065 17.78) (width 0.2) (layer "F.Cu") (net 24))
 (segment (start 3.175 22.86) (end 6.985 19.05) (width 0.2) (layer "F.Cu") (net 24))
 (segment (start -6.35 33.02) (end 0 33.02) (width 0.38) (layer "F.Cu") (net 11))
 (segment (start 21.082 13.462) (end 21.59 13.97) (width 0.2) (layer "F.Cu") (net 5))
 (segment (start 21.59 13.97) (end 30.353 13.97) (width 0.2) (layer "F.Cu") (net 5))
 (segment (start 4.8895 13.97) (end 9.398 13.97) (width 0.2) (layer "F.Cu") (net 5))
 (segment (start 12.827 13.462) (end 13.154 13.789) (width 0.2) (layer "F.Cu") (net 5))
 (segment (start -6.35 15.24) (end -2.54 11.43) (width 0.2) (layer "F.Cu") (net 5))
 (segment (start 9.398 13.97) (end 9.906 13.462) (width 0.2) (layer "F.Cu") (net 5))
 (segment (start 13.154 13.789) (end 15.04 13.789) (width 0.2) (layer "F.Cu") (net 5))
 (segment (start -2.54 11.43) (end 2.3495 11.43) (width 0.2) (layer "F.Cu") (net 5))
 (segment (start 15.367 13.462) (end 21.082 13.462) (width 0.2) (layer "F.Cu") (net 5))
 (segment (start 2.3495 11.43) (end 4.8895 13.97) (width 0.2) (layer "F.Cu") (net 5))
 (segment (start 15.04 13.789) (end 15.367 13.462) (width 0.2) (layer "F.Cu") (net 5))
 (segment (start 9.906 13.462) (end 12.827 13.462) (width 0.2) (layer "F.Cu") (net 5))
 (via (at 30.353 13.97) (size 0.8) (drill 0.4) (layers "F.Cu" "B.Cu") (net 5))
 (segment (start 26.289 29.591) (end 26.289 20.701) (width 0.2) (layer "B.Cu") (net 5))
 (segment (start 30.353 13.97) (end 30.353 16.637) (width 0.2) (layer "B.Cu") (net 5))
 (segment (start 22.86 33.02) (end 26.289 29.591) (width 0.2) (layer "B.Cu") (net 5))
 (segment (start 26.289 20.701) (end 29.21 17.78) (width 0.2) (layer "B.Cu") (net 5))
 (segment (start 30.353 16.637) (end 29.21 17.78) (width 0.2) (layer "B.Cu") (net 5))
 (segment (start 22.86 35.56) (end 27.051 31.369) (width 0.2) (layer "B.Cu") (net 31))
 (segment (start 27.051 22.479) (end 29.21 20.32) (width 0.2) (layer "B.Cu") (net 31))
 (segment (start 27.051 31.369) (end 27.051 22.479) (width 0.2) (layer "B.Cu") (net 31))
 (segment (start 0 12.7) (end -1.27 12.7) (width 0.2) (layer "F.Cu") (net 6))
 (segment (start -1.27 12.7) (end -6.35 17.78) (width 0.2) (layer "F.Cu") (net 6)))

